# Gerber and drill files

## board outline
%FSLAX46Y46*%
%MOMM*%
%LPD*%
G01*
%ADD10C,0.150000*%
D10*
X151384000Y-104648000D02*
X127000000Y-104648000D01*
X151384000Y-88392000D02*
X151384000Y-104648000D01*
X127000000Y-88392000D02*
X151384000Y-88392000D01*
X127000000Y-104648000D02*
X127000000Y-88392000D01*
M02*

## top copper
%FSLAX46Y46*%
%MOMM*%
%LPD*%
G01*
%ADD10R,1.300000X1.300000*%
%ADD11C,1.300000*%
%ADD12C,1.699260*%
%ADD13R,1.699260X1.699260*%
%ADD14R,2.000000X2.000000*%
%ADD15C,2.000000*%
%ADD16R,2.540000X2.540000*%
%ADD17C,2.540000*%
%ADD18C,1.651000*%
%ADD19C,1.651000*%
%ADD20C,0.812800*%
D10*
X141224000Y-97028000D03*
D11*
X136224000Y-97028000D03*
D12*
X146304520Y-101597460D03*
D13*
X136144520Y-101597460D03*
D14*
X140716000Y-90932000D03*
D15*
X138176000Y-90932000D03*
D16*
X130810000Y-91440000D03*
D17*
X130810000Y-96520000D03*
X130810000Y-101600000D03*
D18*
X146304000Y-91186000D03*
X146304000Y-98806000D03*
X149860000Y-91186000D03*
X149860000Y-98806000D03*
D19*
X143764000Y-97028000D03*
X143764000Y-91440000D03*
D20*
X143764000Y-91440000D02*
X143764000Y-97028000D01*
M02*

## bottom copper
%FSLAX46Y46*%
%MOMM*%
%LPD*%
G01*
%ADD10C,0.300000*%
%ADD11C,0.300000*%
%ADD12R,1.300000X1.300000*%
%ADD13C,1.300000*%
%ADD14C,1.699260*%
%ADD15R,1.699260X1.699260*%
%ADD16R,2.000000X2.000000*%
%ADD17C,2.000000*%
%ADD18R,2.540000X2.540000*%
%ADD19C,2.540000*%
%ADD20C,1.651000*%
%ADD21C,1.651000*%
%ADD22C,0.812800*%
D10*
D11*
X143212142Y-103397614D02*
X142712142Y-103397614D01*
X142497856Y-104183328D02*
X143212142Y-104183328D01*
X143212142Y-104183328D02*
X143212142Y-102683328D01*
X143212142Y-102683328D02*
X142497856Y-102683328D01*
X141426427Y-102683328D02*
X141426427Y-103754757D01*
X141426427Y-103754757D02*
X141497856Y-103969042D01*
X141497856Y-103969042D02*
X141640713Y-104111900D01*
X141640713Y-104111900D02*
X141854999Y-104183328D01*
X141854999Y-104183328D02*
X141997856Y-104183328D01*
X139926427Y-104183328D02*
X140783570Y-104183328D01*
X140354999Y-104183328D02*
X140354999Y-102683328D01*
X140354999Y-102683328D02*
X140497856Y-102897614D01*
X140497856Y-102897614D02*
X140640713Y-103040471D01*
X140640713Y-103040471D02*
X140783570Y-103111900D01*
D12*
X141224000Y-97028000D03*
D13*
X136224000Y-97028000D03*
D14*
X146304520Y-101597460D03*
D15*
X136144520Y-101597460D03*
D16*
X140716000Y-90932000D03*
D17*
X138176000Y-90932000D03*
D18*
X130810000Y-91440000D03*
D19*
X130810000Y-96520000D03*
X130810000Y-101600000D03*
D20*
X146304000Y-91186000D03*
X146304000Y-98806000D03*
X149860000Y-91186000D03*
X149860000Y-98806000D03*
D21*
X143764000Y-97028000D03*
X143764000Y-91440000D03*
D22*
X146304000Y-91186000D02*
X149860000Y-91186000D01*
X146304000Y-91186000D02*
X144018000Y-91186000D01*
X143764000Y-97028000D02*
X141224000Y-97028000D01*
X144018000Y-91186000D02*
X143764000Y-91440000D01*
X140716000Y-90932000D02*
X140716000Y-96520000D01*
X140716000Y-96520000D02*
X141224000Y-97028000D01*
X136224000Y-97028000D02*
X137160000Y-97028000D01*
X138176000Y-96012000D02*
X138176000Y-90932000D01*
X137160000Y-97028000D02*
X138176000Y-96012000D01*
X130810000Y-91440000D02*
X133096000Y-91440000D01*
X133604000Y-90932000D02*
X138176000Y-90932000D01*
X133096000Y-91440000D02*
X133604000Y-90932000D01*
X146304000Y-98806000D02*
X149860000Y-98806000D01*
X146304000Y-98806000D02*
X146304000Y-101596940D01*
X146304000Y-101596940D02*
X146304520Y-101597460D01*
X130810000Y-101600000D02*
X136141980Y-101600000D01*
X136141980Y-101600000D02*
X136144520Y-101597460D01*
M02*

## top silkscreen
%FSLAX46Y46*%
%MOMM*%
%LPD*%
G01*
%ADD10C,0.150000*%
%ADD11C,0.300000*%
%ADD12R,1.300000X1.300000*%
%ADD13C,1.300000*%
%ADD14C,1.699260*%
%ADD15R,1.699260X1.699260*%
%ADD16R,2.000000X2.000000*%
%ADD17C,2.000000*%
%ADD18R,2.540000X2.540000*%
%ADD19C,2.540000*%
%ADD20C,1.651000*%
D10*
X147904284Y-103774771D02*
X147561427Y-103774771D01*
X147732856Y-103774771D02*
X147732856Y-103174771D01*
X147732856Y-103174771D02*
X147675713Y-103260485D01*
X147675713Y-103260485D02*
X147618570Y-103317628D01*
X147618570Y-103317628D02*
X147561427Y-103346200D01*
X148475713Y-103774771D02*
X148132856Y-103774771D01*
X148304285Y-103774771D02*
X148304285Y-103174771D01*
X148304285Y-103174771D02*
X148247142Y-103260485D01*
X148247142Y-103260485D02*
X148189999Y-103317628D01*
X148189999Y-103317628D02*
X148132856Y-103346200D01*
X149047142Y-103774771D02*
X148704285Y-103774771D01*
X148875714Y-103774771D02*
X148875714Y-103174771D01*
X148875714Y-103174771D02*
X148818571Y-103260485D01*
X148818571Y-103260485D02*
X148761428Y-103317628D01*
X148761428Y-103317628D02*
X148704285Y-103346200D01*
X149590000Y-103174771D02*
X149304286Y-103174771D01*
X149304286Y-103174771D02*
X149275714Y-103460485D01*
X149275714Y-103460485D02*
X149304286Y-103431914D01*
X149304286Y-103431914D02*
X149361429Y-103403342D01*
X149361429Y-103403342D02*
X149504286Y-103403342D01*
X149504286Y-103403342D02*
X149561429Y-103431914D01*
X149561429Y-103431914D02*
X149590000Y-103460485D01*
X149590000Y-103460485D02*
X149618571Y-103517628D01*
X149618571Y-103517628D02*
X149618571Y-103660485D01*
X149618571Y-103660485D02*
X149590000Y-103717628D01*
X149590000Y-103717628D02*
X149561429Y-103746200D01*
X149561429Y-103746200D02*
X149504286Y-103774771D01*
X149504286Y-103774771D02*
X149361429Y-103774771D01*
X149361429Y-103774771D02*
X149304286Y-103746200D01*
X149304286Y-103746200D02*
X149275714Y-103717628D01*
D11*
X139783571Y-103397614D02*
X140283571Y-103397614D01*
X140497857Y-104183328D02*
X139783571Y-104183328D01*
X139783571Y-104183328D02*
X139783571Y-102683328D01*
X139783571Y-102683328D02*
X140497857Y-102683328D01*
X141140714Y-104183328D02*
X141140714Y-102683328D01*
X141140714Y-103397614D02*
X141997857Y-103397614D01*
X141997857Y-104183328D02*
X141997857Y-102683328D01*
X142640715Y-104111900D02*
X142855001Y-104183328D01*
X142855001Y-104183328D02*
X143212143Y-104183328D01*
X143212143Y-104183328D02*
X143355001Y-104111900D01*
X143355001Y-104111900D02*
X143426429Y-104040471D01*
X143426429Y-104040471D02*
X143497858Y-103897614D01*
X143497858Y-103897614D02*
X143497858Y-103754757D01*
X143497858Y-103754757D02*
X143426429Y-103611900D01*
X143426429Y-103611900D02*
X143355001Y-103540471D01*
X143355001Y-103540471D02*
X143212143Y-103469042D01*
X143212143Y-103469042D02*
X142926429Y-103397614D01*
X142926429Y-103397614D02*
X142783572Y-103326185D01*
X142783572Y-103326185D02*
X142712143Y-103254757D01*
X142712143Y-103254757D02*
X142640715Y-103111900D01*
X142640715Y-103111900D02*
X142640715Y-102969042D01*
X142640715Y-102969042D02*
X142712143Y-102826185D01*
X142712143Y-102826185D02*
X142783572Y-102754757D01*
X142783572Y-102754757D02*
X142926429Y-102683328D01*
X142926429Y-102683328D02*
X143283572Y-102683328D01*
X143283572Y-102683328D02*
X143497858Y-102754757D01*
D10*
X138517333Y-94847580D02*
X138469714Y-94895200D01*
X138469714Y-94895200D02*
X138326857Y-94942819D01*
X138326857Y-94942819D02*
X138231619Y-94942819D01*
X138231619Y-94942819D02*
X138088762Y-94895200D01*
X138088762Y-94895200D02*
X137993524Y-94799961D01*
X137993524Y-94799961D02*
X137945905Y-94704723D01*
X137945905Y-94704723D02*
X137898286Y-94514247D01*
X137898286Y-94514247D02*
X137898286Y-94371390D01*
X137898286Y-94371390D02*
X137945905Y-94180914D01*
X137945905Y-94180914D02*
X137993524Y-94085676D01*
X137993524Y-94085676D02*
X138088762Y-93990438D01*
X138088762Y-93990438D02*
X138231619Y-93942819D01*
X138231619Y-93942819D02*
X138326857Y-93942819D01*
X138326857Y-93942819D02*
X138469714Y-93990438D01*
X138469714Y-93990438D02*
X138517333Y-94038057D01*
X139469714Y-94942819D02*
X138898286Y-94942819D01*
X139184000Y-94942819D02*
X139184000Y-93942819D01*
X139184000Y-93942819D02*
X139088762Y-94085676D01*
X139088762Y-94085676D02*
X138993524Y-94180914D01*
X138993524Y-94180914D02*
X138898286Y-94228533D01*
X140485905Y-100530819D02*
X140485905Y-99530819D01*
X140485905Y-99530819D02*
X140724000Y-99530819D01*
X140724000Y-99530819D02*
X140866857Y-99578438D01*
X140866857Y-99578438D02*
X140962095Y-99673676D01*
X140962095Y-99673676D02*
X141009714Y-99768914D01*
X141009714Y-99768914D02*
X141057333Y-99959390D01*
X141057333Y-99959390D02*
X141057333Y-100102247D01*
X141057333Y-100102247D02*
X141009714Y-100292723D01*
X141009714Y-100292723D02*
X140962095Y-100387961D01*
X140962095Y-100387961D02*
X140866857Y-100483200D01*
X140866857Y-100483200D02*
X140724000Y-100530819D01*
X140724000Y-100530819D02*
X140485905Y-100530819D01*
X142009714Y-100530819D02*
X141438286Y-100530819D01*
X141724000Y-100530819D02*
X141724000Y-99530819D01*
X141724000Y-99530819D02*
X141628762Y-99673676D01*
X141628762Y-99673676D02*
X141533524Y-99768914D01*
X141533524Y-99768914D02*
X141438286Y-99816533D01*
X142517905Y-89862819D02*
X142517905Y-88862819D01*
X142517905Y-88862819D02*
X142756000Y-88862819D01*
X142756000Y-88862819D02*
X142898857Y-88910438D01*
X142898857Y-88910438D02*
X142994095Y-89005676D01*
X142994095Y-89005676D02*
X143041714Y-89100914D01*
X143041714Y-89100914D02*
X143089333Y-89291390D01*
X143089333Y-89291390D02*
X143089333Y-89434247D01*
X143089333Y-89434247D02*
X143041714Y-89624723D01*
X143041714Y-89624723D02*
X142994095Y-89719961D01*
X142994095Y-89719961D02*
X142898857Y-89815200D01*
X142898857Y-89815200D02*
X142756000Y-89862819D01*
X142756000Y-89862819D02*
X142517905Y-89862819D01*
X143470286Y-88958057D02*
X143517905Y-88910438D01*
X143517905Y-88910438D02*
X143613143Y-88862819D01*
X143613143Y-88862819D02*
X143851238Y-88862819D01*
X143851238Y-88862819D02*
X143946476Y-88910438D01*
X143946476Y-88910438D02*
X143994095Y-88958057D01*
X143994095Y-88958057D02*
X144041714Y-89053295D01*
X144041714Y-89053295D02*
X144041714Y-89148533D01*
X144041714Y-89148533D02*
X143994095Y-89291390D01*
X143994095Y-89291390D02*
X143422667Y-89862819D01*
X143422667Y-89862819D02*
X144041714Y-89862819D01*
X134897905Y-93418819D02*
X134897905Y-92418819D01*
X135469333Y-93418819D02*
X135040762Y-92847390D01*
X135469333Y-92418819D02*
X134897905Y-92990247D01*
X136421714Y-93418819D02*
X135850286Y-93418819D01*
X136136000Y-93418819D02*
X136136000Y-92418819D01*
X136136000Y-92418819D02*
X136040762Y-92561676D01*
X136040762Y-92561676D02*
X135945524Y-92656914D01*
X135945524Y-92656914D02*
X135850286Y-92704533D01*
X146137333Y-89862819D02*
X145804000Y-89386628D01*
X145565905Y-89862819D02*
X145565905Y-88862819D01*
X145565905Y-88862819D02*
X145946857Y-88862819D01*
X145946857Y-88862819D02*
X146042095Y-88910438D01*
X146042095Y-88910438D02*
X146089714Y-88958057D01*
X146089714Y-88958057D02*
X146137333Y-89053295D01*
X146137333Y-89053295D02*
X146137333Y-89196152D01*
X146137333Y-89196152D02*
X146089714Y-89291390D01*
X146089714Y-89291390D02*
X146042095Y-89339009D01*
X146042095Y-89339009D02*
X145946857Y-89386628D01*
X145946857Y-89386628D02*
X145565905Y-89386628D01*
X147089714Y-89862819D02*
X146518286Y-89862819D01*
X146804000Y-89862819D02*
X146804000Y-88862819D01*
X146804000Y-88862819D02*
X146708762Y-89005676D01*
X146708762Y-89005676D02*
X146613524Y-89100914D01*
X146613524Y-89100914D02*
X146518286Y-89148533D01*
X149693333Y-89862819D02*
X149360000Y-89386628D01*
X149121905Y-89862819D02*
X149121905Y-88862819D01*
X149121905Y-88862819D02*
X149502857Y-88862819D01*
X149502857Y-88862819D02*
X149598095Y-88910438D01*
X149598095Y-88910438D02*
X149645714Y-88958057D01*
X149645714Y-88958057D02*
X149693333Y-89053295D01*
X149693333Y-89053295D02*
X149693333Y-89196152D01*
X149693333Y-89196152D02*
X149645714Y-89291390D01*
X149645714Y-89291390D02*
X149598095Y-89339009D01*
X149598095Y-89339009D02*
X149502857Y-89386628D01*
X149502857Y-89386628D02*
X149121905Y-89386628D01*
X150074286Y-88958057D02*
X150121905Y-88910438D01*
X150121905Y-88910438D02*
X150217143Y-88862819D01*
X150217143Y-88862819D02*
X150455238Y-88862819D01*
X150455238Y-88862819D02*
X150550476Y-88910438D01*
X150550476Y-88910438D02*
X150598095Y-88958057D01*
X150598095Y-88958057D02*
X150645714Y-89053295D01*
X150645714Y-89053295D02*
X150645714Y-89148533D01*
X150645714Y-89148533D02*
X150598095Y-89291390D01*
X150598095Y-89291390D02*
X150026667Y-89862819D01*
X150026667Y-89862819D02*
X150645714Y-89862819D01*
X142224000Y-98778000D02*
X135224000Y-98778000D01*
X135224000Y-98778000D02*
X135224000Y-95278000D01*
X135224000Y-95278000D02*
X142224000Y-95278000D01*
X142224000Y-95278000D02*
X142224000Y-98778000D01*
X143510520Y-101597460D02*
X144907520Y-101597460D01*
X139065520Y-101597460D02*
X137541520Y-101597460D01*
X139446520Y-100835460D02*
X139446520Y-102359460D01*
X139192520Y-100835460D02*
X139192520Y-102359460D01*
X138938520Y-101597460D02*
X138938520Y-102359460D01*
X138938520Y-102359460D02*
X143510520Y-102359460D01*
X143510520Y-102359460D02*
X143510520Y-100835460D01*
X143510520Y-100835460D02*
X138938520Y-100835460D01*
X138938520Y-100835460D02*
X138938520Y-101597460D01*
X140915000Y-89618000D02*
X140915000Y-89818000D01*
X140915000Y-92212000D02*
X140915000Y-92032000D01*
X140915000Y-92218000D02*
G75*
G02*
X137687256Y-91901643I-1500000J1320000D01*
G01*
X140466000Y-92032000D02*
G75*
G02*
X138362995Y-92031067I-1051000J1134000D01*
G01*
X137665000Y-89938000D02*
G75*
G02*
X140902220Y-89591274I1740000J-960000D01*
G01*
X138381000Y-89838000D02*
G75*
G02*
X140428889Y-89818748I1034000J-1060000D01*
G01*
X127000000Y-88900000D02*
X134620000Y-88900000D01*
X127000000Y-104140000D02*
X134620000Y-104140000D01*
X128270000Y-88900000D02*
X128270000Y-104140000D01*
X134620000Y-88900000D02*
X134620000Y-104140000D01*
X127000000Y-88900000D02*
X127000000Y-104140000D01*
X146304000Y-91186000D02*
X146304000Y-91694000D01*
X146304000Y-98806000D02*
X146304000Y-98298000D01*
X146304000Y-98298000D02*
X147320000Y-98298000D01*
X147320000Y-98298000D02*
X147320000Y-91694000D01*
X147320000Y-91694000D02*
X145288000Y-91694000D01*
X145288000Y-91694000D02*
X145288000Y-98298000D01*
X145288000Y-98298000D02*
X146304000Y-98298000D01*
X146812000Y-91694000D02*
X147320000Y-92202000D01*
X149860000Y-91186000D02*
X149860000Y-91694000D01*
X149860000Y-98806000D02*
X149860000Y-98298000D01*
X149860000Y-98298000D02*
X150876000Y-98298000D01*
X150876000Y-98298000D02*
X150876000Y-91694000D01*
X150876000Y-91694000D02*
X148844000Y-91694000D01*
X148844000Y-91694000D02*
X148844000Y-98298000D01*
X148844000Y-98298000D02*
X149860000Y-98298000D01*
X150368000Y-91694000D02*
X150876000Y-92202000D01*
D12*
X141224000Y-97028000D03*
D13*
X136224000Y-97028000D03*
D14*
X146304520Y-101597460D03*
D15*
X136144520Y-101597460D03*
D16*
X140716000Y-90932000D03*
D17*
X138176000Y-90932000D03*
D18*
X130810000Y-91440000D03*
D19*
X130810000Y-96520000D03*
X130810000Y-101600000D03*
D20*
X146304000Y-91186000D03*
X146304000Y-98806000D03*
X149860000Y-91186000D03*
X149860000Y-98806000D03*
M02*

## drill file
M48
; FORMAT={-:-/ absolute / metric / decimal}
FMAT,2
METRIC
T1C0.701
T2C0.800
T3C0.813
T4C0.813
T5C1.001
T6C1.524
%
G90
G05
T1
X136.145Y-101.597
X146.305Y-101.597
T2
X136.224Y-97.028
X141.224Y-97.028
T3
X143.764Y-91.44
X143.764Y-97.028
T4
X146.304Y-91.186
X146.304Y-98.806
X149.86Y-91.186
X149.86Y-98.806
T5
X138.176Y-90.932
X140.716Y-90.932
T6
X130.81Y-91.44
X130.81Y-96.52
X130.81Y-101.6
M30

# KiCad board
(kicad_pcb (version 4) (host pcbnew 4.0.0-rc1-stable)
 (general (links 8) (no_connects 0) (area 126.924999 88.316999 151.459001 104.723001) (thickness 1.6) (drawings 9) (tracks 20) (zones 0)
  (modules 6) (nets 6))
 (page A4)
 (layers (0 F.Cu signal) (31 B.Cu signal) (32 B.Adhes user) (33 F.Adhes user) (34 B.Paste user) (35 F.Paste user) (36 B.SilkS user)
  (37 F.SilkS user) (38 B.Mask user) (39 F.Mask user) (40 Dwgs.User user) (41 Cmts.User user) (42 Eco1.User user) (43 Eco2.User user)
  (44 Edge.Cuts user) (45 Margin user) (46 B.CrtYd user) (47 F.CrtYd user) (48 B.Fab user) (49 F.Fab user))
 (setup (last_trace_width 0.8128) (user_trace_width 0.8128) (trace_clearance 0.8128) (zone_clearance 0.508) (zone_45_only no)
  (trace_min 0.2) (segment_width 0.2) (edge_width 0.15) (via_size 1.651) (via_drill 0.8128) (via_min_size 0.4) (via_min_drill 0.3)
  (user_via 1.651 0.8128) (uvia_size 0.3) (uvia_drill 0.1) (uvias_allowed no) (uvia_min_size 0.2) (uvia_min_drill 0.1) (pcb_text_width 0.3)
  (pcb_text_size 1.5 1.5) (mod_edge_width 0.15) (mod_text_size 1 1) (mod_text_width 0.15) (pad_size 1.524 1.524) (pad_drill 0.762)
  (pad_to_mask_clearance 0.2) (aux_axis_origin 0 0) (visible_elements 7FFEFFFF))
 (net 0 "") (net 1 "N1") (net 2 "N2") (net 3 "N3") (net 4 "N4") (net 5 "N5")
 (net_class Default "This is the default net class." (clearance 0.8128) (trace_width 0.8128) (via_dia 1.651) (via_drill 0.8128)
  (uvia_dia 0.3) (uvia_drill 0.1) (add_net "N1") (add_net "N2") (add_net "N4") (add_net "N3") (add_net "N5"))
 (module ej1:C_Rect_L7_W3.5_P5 (layer F.Cu) (at 141.224 97.028 180)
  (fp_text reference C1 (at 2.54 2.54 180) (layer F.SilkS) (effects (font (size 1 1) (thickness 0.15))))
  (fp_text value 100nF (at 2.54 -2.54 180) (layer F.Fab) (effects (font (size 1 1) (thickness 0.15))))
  (fp_line (start -1 -1.75) (end 6 -1.75) (layer F.SilkS) (width 0.15))
  (fp_line (start 6 -1.75) (end 6 1.75) (layer F.SilkS) (width 0.15))
  (fp_line (start 6 1.75) (end -1 1.75) (layer F.SilkS) (width 0.15))
  (fp_line (start -1 1.75) (end -1 -1.75) (layer F.SilkS) (width 0.15))
  (pad 1 thru_hole rect (at 0 0 180) (size 1.3 1.3) (drill 0.8) (layers *.Cu *.Mask F.SilkS) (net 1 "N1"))
  (pad 2 thru_hole circle (at 5 0 180) (size 1.3 1.3) (drill 0.8) (layers *.Cu *.Mask F.SilkS) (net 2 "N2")))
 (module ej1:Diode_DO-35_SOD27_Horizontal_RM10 (layer F.Cu) (at 136.144 101.6)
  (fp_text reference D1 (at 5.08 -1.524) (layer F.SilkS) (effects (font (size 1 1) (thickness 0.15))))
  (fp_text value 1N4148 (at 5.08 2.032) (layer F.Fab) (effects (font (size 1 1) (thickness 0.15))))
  (fp_line (start 7.36652 -0.00254) (end 8.76352 -0.00254) (layer F.SilkS) (width 0.15))
  (fp_line (start 2.92152 -0.00254) (end 1.39752 -0.00254) (layer F.SilkS) (width 0.15))
  (fp_line (start 3.30252 -0.76454) (end 3.30252 0.75946) (layer F.SilkS) (width 0.15))
  (fp_line (start 3.04852 -0.76454) (end 3.04852 0.75946) (layer F.SilkS) (width 0.15))
  (fp_line (start 2.79452 -0.00254) (end 2.79452 0.75946) (layer F.SilkS) (width 0.15))
  (fp_line (start 2.79452 0.75946) (end 7.36652 0.75946) (layer F.SilkS) (width 0.15))
  (fp_line (start 7.36652 0.75946) (end 7.36652 -0.76454) (layer F.SilkS) (width 0.15))
  (fp_line (start 7.36652 -0.76454) (end 2.79452 -0.76454) (layer F.SilkS) (width 0.15))
  (fp_line (start 2.79452 -0.76454) (end 2.79452 -0.00254) (layer F.SilkS) (width 0.15))
  (pad 2 thru_hole circle (at 10.16052 -0.00254 180) (size 1.69926 1.69926) (drill 0.70104) (layers *.Cu *.Mask F.SilkS) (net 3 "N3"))
  (pad 1 thru_hole rect (at 0.00052 -0.00254 180) (size 1.69926 1.69926) (drill 0.70104) (layers *.Cu *.Mask F.SilkS) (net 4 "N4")))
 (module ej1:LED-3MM (layer F.Cu) (at 140.716 90.932 180)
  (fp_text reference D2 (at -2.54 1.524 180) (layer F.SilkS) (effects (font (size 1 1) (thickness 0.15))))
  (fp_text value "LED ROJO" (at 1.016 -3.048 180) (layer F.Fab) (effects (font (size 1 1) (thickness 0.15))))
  (fp_line (start -0.199 1.314) (end -0.199 1.114) (layer F.SilkS) (width 0.15))
  (fp_line (start -0.199 -1.28) (end -0.199 -1.1) (layer F.SilkS) (width 0.15))
  (fp_arc (start 1.301 0.034) (end -0.199 -1.286) (angle 108.5) (layer F.SilkS) (width 0.15))
  (fp_arc (start 1.301 0.034) (end 0.25 -1.1) (angle 85.7) (layer F.SilkS) (width 0.15))
  (fp_arc (start 1.311 0.034) (end 3.051 0.994) (angle 110) (layer F.SilkS) (width 0.15))
  (fp_arc (start 1.301 0.034) (end 2.335 1.094) (angle 87.5) (layer F.SilkS) (width 0.15))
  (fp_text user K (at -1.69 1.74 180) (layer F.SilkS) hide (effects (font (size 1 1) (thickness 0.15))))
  (pad 1 thru_hole rect (at 0 0 270) (size 2 2) (drill 1.00076) (layers *.Cu *.Mask F.SilkS) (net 1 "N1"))
  (pad 2 thru_hole circle (at 2.54 0 180) (size 2 2) (drill 1.00076) (layers *.Cu *.Mask F.SilkS) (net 2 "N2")))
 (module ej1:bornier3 (layer F.Cu) (at 130.81 96.52 270)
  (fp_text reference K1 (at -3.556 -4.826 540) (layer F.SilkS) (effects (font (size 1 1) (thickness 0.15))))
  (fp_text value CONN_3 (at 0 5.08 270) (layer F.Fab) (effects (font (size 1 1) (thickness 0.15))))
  (fp_line (start -7.62 3.81) (end -7.62 -3.81) (layer F.SilkS) (width 0.15))
  (fp_line (start 7.62 3.81) (end 7.62 -3.81) (layer F.SilkS) (width 0.15))
  (fp_line (start -7.62 2.54) (end 7.62 2.54) (layer F.SilkS) (width 0.15))
  (fp_line (start -7.62 -3.81) (end 7.62 -3.81) (layer F.SilkS) (width 0.15))
  (fp_line (start -7.62 3.81) (end 7.62 3.81) (layer F.SilkS) (width 0.15))
  (pad 1 thru_hole rect (at -5.08 0 270) (size 2.54 2.54) (drill 1.524) (layers *.Cu *.Mask F.SilkS) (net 2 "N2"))
  (pad 2 thru_hole circle (at 0 0 270) (size 2.54 2.54) (drill 1.524) (layers *.Cu *.Mask F.SilkS) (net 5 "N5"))
  (pad 3 thru_hole circle (at 5.08 0 270) (size 2.54 2.54) (drill 1.524) (layers *.Cu *.Mask F.SilkS) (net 4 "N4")))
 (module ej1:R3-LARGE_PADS (layer F.Cu) (at 146.304 94.996 270)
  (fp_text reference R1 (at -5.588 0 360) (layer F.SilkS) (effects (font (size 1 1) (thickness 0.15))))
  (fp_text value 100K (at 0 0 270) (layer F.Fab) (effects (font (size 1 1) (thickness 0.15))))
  (fp_line (start -3.81 0) (end -3.302 0) (layer F.SilkS) (width 0.15))
  (fp_line (start 3.81 0) (end 3.302 0) (layer F.SilkS) (width 0.15))
  (fp_line (start 3.302 0) (end 3.302 -1.016) (layer F.SilkS) (width 0.15))
  (fp_line (start 3.302 -1.016) (end -3.302 -1.016) (layer F.SilkS) (width 0.15))
  (fp_line (start -3.302 -1.016) (end -3.302 1.016) (layer F.SilkS) (width 0.15))
  (fp_line (start -3.302 1.016) (end 3.302 1.016) (layer F.SilkS) (width 0.15))
  (fp_line (start 3.302 1.016) (end 3.302 0) (layer F.SilkS) (width 0.15))
  (fp_line (start -3.302 -0.508) (end -2.794 -1.016) (layer F.SilkS) (width 0.15))
  (pad 1 thru_hole circle (at -3.81 0 270) (size 1.651 1.651) (drill 0.8128) (layers *.Cu *.Mask F.SilkS) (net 1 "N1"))
  (pad 2 thru_hole circle (at 3.81 0 270) (size 1.651 1.651) (drill 0.8128) (layers *.Cu *.Mask F.SilkS) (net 3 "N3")))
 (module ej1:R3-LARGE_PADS (layer F.Cu) (at 149.86 94.996 270)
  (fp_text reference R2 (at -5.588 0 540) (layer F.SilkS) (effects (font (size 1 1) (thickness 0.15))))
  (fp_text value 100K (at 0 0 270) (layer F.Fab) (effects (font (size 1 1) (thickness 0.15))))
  (fp_line (start -3.81 0) (end -3.302 0) (layer F.SilkS) (width 0.15))
  (fp_line (start 3.81 0) (end 3.302 0) (layer F.SilkS) (width 0.15))
  (fp_line (start 3.302 0) (end 3.302 -1.016) (layer F.SilkS) (width 0.15))
  (fp_line (start 3.302 -1.016) (end -3.302 -1.016) (layer F.SilkS) (width 0.15))
  (fp_line (start -3.302 -1.016) (end -3.302 1.016) (layer F.SilkS) (width 0.15))
  (fp_line (start -3.302 1.016) (end 3.302 1.016) (layer F.SilkS) (width 0.15))
  (fp_line (start 3.302 1.016) (end 3.302 0) (layer F.SilkS) (width 0.15))
  (fp_line (start -3.302 -0.508) (end -2.794 -1.016) (layer F.SilkS) (width 0.15))
  (pad 1 thru_hole circle (at -3.81 0 270) (size 1.651 1.651) (drill 0.8128) (layers *.Cu *.Mask F.SilkS) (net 1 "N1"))
  (pad 2 thru_hole circle (at 3.81 0 270) (size 1.651 1.651) (drill 0.8128) (layers *.Cu *.Mask F.SilkS) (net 3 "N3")))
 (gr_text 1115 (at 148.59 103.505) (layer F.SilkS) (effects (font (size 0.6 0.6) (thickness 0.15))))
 (gr_line (start 151.384 104.648) (end 127 104.648) (angle 90) (layer Edge.Cuts) (width 0.15))
 (gr_line (start 151.384 88.392) (end 151.384 104.648) (angle 90) (layer Edge.Cuts) (width 0.15))
 (gr_line (start 127 88.392) (end 151.384 88.392) (angle 90) (layer Edge.Cuts) (width 0.15))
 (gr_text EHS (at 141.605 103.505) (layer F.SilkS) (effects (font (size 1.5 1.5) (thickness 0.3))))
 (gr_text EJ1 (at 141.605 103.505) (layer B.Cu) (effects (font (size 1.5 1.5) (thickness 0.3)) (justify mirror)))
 (gr_line (start 127 104.648) (end 127 88.392) (angle 90) (layer Edge.Cuts) (width 0.15))
 (segment (start 146.304 91.186) (end 149.86 91.186) (width 0.8128) (layer B.Cu) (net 1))
 (segment (start 146.304 91.186) (end 144.018 91.186) (width 0.8128) (layer B.Cu) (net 1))
 (segment (start 143.764 97.028) (end 141.224 97.028) (width 0.8128) (layer B.Cu) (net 1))
 (via (at 143.764 97.028) (size 1.651) (drill 0.8128) (layers F.Cu B.Cu) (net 1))
 (segment (start 143.764 91.44) (end 143.764 97.028) (width 0.8128) (layer F.Cu) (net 1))
 (via (at 143.764 91.44) (size 1.651) (drill 0.8128) (layers F.Cu B.Cu) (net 1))
 (segment (start 144.018 91.186) (end 143.764 91.44) (width 0.8128) (layer B.Cu) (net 1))
 (segment (start 140.716 90.932) (end 140.716 96.52) (width 0.8128) (layer B.Cu) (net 1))
 (segment (start 140.716 96.52) (end 141.224 97.028) (width 0.8128) (layer B.Cu) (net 1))
 (segment (start 136.224 97.028) (end 137.16 97.028) (width 0.8128) (layer B.Cu) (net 2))
 (segment (start 138.176 96.012) (end 138.176 90.932) (width 0.8128) (layer B.Cu) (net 2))
 (segment (start 137.16 97.028) (end 138.176 96.012) (width 0.8128) (layer B.Cu) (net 2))
 (segment (start 130.81 91.44) (end 133.096 91.44) (width 0.8128) (layer B.Cu) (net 2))
 (segment (start 133.604 90.932) (end 138.176 90.932) (width 0.8128) (layer B.Cu) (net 2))
 (segment (start 133.096 91.44) (end 133.604 90.932) (width 0.8128) (layer B.Cu) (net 2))
 (segment (start 146.304 98.806) (end 149.86 98.806) (width 0.8128) (layer B.Cu) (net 3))
 (segment (start 146.304 98.806) (end 146.304 101.59694) (width 0.8128) (layer B.Cu) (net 3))
 (segment (start 146.304 101.59694) (end 146.30452 101.59746) (width 0.8128) (layer B.Cu) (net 3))
 (segment (start 130.81 101.6) (end 136.14198 101.6) (width 0.8128) (layer B.Cu) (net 4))
 (segment (start 136.14198 101.6) (end 136.14452 101.59746) (width 0.8128) (layer B.Cu) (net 4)))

